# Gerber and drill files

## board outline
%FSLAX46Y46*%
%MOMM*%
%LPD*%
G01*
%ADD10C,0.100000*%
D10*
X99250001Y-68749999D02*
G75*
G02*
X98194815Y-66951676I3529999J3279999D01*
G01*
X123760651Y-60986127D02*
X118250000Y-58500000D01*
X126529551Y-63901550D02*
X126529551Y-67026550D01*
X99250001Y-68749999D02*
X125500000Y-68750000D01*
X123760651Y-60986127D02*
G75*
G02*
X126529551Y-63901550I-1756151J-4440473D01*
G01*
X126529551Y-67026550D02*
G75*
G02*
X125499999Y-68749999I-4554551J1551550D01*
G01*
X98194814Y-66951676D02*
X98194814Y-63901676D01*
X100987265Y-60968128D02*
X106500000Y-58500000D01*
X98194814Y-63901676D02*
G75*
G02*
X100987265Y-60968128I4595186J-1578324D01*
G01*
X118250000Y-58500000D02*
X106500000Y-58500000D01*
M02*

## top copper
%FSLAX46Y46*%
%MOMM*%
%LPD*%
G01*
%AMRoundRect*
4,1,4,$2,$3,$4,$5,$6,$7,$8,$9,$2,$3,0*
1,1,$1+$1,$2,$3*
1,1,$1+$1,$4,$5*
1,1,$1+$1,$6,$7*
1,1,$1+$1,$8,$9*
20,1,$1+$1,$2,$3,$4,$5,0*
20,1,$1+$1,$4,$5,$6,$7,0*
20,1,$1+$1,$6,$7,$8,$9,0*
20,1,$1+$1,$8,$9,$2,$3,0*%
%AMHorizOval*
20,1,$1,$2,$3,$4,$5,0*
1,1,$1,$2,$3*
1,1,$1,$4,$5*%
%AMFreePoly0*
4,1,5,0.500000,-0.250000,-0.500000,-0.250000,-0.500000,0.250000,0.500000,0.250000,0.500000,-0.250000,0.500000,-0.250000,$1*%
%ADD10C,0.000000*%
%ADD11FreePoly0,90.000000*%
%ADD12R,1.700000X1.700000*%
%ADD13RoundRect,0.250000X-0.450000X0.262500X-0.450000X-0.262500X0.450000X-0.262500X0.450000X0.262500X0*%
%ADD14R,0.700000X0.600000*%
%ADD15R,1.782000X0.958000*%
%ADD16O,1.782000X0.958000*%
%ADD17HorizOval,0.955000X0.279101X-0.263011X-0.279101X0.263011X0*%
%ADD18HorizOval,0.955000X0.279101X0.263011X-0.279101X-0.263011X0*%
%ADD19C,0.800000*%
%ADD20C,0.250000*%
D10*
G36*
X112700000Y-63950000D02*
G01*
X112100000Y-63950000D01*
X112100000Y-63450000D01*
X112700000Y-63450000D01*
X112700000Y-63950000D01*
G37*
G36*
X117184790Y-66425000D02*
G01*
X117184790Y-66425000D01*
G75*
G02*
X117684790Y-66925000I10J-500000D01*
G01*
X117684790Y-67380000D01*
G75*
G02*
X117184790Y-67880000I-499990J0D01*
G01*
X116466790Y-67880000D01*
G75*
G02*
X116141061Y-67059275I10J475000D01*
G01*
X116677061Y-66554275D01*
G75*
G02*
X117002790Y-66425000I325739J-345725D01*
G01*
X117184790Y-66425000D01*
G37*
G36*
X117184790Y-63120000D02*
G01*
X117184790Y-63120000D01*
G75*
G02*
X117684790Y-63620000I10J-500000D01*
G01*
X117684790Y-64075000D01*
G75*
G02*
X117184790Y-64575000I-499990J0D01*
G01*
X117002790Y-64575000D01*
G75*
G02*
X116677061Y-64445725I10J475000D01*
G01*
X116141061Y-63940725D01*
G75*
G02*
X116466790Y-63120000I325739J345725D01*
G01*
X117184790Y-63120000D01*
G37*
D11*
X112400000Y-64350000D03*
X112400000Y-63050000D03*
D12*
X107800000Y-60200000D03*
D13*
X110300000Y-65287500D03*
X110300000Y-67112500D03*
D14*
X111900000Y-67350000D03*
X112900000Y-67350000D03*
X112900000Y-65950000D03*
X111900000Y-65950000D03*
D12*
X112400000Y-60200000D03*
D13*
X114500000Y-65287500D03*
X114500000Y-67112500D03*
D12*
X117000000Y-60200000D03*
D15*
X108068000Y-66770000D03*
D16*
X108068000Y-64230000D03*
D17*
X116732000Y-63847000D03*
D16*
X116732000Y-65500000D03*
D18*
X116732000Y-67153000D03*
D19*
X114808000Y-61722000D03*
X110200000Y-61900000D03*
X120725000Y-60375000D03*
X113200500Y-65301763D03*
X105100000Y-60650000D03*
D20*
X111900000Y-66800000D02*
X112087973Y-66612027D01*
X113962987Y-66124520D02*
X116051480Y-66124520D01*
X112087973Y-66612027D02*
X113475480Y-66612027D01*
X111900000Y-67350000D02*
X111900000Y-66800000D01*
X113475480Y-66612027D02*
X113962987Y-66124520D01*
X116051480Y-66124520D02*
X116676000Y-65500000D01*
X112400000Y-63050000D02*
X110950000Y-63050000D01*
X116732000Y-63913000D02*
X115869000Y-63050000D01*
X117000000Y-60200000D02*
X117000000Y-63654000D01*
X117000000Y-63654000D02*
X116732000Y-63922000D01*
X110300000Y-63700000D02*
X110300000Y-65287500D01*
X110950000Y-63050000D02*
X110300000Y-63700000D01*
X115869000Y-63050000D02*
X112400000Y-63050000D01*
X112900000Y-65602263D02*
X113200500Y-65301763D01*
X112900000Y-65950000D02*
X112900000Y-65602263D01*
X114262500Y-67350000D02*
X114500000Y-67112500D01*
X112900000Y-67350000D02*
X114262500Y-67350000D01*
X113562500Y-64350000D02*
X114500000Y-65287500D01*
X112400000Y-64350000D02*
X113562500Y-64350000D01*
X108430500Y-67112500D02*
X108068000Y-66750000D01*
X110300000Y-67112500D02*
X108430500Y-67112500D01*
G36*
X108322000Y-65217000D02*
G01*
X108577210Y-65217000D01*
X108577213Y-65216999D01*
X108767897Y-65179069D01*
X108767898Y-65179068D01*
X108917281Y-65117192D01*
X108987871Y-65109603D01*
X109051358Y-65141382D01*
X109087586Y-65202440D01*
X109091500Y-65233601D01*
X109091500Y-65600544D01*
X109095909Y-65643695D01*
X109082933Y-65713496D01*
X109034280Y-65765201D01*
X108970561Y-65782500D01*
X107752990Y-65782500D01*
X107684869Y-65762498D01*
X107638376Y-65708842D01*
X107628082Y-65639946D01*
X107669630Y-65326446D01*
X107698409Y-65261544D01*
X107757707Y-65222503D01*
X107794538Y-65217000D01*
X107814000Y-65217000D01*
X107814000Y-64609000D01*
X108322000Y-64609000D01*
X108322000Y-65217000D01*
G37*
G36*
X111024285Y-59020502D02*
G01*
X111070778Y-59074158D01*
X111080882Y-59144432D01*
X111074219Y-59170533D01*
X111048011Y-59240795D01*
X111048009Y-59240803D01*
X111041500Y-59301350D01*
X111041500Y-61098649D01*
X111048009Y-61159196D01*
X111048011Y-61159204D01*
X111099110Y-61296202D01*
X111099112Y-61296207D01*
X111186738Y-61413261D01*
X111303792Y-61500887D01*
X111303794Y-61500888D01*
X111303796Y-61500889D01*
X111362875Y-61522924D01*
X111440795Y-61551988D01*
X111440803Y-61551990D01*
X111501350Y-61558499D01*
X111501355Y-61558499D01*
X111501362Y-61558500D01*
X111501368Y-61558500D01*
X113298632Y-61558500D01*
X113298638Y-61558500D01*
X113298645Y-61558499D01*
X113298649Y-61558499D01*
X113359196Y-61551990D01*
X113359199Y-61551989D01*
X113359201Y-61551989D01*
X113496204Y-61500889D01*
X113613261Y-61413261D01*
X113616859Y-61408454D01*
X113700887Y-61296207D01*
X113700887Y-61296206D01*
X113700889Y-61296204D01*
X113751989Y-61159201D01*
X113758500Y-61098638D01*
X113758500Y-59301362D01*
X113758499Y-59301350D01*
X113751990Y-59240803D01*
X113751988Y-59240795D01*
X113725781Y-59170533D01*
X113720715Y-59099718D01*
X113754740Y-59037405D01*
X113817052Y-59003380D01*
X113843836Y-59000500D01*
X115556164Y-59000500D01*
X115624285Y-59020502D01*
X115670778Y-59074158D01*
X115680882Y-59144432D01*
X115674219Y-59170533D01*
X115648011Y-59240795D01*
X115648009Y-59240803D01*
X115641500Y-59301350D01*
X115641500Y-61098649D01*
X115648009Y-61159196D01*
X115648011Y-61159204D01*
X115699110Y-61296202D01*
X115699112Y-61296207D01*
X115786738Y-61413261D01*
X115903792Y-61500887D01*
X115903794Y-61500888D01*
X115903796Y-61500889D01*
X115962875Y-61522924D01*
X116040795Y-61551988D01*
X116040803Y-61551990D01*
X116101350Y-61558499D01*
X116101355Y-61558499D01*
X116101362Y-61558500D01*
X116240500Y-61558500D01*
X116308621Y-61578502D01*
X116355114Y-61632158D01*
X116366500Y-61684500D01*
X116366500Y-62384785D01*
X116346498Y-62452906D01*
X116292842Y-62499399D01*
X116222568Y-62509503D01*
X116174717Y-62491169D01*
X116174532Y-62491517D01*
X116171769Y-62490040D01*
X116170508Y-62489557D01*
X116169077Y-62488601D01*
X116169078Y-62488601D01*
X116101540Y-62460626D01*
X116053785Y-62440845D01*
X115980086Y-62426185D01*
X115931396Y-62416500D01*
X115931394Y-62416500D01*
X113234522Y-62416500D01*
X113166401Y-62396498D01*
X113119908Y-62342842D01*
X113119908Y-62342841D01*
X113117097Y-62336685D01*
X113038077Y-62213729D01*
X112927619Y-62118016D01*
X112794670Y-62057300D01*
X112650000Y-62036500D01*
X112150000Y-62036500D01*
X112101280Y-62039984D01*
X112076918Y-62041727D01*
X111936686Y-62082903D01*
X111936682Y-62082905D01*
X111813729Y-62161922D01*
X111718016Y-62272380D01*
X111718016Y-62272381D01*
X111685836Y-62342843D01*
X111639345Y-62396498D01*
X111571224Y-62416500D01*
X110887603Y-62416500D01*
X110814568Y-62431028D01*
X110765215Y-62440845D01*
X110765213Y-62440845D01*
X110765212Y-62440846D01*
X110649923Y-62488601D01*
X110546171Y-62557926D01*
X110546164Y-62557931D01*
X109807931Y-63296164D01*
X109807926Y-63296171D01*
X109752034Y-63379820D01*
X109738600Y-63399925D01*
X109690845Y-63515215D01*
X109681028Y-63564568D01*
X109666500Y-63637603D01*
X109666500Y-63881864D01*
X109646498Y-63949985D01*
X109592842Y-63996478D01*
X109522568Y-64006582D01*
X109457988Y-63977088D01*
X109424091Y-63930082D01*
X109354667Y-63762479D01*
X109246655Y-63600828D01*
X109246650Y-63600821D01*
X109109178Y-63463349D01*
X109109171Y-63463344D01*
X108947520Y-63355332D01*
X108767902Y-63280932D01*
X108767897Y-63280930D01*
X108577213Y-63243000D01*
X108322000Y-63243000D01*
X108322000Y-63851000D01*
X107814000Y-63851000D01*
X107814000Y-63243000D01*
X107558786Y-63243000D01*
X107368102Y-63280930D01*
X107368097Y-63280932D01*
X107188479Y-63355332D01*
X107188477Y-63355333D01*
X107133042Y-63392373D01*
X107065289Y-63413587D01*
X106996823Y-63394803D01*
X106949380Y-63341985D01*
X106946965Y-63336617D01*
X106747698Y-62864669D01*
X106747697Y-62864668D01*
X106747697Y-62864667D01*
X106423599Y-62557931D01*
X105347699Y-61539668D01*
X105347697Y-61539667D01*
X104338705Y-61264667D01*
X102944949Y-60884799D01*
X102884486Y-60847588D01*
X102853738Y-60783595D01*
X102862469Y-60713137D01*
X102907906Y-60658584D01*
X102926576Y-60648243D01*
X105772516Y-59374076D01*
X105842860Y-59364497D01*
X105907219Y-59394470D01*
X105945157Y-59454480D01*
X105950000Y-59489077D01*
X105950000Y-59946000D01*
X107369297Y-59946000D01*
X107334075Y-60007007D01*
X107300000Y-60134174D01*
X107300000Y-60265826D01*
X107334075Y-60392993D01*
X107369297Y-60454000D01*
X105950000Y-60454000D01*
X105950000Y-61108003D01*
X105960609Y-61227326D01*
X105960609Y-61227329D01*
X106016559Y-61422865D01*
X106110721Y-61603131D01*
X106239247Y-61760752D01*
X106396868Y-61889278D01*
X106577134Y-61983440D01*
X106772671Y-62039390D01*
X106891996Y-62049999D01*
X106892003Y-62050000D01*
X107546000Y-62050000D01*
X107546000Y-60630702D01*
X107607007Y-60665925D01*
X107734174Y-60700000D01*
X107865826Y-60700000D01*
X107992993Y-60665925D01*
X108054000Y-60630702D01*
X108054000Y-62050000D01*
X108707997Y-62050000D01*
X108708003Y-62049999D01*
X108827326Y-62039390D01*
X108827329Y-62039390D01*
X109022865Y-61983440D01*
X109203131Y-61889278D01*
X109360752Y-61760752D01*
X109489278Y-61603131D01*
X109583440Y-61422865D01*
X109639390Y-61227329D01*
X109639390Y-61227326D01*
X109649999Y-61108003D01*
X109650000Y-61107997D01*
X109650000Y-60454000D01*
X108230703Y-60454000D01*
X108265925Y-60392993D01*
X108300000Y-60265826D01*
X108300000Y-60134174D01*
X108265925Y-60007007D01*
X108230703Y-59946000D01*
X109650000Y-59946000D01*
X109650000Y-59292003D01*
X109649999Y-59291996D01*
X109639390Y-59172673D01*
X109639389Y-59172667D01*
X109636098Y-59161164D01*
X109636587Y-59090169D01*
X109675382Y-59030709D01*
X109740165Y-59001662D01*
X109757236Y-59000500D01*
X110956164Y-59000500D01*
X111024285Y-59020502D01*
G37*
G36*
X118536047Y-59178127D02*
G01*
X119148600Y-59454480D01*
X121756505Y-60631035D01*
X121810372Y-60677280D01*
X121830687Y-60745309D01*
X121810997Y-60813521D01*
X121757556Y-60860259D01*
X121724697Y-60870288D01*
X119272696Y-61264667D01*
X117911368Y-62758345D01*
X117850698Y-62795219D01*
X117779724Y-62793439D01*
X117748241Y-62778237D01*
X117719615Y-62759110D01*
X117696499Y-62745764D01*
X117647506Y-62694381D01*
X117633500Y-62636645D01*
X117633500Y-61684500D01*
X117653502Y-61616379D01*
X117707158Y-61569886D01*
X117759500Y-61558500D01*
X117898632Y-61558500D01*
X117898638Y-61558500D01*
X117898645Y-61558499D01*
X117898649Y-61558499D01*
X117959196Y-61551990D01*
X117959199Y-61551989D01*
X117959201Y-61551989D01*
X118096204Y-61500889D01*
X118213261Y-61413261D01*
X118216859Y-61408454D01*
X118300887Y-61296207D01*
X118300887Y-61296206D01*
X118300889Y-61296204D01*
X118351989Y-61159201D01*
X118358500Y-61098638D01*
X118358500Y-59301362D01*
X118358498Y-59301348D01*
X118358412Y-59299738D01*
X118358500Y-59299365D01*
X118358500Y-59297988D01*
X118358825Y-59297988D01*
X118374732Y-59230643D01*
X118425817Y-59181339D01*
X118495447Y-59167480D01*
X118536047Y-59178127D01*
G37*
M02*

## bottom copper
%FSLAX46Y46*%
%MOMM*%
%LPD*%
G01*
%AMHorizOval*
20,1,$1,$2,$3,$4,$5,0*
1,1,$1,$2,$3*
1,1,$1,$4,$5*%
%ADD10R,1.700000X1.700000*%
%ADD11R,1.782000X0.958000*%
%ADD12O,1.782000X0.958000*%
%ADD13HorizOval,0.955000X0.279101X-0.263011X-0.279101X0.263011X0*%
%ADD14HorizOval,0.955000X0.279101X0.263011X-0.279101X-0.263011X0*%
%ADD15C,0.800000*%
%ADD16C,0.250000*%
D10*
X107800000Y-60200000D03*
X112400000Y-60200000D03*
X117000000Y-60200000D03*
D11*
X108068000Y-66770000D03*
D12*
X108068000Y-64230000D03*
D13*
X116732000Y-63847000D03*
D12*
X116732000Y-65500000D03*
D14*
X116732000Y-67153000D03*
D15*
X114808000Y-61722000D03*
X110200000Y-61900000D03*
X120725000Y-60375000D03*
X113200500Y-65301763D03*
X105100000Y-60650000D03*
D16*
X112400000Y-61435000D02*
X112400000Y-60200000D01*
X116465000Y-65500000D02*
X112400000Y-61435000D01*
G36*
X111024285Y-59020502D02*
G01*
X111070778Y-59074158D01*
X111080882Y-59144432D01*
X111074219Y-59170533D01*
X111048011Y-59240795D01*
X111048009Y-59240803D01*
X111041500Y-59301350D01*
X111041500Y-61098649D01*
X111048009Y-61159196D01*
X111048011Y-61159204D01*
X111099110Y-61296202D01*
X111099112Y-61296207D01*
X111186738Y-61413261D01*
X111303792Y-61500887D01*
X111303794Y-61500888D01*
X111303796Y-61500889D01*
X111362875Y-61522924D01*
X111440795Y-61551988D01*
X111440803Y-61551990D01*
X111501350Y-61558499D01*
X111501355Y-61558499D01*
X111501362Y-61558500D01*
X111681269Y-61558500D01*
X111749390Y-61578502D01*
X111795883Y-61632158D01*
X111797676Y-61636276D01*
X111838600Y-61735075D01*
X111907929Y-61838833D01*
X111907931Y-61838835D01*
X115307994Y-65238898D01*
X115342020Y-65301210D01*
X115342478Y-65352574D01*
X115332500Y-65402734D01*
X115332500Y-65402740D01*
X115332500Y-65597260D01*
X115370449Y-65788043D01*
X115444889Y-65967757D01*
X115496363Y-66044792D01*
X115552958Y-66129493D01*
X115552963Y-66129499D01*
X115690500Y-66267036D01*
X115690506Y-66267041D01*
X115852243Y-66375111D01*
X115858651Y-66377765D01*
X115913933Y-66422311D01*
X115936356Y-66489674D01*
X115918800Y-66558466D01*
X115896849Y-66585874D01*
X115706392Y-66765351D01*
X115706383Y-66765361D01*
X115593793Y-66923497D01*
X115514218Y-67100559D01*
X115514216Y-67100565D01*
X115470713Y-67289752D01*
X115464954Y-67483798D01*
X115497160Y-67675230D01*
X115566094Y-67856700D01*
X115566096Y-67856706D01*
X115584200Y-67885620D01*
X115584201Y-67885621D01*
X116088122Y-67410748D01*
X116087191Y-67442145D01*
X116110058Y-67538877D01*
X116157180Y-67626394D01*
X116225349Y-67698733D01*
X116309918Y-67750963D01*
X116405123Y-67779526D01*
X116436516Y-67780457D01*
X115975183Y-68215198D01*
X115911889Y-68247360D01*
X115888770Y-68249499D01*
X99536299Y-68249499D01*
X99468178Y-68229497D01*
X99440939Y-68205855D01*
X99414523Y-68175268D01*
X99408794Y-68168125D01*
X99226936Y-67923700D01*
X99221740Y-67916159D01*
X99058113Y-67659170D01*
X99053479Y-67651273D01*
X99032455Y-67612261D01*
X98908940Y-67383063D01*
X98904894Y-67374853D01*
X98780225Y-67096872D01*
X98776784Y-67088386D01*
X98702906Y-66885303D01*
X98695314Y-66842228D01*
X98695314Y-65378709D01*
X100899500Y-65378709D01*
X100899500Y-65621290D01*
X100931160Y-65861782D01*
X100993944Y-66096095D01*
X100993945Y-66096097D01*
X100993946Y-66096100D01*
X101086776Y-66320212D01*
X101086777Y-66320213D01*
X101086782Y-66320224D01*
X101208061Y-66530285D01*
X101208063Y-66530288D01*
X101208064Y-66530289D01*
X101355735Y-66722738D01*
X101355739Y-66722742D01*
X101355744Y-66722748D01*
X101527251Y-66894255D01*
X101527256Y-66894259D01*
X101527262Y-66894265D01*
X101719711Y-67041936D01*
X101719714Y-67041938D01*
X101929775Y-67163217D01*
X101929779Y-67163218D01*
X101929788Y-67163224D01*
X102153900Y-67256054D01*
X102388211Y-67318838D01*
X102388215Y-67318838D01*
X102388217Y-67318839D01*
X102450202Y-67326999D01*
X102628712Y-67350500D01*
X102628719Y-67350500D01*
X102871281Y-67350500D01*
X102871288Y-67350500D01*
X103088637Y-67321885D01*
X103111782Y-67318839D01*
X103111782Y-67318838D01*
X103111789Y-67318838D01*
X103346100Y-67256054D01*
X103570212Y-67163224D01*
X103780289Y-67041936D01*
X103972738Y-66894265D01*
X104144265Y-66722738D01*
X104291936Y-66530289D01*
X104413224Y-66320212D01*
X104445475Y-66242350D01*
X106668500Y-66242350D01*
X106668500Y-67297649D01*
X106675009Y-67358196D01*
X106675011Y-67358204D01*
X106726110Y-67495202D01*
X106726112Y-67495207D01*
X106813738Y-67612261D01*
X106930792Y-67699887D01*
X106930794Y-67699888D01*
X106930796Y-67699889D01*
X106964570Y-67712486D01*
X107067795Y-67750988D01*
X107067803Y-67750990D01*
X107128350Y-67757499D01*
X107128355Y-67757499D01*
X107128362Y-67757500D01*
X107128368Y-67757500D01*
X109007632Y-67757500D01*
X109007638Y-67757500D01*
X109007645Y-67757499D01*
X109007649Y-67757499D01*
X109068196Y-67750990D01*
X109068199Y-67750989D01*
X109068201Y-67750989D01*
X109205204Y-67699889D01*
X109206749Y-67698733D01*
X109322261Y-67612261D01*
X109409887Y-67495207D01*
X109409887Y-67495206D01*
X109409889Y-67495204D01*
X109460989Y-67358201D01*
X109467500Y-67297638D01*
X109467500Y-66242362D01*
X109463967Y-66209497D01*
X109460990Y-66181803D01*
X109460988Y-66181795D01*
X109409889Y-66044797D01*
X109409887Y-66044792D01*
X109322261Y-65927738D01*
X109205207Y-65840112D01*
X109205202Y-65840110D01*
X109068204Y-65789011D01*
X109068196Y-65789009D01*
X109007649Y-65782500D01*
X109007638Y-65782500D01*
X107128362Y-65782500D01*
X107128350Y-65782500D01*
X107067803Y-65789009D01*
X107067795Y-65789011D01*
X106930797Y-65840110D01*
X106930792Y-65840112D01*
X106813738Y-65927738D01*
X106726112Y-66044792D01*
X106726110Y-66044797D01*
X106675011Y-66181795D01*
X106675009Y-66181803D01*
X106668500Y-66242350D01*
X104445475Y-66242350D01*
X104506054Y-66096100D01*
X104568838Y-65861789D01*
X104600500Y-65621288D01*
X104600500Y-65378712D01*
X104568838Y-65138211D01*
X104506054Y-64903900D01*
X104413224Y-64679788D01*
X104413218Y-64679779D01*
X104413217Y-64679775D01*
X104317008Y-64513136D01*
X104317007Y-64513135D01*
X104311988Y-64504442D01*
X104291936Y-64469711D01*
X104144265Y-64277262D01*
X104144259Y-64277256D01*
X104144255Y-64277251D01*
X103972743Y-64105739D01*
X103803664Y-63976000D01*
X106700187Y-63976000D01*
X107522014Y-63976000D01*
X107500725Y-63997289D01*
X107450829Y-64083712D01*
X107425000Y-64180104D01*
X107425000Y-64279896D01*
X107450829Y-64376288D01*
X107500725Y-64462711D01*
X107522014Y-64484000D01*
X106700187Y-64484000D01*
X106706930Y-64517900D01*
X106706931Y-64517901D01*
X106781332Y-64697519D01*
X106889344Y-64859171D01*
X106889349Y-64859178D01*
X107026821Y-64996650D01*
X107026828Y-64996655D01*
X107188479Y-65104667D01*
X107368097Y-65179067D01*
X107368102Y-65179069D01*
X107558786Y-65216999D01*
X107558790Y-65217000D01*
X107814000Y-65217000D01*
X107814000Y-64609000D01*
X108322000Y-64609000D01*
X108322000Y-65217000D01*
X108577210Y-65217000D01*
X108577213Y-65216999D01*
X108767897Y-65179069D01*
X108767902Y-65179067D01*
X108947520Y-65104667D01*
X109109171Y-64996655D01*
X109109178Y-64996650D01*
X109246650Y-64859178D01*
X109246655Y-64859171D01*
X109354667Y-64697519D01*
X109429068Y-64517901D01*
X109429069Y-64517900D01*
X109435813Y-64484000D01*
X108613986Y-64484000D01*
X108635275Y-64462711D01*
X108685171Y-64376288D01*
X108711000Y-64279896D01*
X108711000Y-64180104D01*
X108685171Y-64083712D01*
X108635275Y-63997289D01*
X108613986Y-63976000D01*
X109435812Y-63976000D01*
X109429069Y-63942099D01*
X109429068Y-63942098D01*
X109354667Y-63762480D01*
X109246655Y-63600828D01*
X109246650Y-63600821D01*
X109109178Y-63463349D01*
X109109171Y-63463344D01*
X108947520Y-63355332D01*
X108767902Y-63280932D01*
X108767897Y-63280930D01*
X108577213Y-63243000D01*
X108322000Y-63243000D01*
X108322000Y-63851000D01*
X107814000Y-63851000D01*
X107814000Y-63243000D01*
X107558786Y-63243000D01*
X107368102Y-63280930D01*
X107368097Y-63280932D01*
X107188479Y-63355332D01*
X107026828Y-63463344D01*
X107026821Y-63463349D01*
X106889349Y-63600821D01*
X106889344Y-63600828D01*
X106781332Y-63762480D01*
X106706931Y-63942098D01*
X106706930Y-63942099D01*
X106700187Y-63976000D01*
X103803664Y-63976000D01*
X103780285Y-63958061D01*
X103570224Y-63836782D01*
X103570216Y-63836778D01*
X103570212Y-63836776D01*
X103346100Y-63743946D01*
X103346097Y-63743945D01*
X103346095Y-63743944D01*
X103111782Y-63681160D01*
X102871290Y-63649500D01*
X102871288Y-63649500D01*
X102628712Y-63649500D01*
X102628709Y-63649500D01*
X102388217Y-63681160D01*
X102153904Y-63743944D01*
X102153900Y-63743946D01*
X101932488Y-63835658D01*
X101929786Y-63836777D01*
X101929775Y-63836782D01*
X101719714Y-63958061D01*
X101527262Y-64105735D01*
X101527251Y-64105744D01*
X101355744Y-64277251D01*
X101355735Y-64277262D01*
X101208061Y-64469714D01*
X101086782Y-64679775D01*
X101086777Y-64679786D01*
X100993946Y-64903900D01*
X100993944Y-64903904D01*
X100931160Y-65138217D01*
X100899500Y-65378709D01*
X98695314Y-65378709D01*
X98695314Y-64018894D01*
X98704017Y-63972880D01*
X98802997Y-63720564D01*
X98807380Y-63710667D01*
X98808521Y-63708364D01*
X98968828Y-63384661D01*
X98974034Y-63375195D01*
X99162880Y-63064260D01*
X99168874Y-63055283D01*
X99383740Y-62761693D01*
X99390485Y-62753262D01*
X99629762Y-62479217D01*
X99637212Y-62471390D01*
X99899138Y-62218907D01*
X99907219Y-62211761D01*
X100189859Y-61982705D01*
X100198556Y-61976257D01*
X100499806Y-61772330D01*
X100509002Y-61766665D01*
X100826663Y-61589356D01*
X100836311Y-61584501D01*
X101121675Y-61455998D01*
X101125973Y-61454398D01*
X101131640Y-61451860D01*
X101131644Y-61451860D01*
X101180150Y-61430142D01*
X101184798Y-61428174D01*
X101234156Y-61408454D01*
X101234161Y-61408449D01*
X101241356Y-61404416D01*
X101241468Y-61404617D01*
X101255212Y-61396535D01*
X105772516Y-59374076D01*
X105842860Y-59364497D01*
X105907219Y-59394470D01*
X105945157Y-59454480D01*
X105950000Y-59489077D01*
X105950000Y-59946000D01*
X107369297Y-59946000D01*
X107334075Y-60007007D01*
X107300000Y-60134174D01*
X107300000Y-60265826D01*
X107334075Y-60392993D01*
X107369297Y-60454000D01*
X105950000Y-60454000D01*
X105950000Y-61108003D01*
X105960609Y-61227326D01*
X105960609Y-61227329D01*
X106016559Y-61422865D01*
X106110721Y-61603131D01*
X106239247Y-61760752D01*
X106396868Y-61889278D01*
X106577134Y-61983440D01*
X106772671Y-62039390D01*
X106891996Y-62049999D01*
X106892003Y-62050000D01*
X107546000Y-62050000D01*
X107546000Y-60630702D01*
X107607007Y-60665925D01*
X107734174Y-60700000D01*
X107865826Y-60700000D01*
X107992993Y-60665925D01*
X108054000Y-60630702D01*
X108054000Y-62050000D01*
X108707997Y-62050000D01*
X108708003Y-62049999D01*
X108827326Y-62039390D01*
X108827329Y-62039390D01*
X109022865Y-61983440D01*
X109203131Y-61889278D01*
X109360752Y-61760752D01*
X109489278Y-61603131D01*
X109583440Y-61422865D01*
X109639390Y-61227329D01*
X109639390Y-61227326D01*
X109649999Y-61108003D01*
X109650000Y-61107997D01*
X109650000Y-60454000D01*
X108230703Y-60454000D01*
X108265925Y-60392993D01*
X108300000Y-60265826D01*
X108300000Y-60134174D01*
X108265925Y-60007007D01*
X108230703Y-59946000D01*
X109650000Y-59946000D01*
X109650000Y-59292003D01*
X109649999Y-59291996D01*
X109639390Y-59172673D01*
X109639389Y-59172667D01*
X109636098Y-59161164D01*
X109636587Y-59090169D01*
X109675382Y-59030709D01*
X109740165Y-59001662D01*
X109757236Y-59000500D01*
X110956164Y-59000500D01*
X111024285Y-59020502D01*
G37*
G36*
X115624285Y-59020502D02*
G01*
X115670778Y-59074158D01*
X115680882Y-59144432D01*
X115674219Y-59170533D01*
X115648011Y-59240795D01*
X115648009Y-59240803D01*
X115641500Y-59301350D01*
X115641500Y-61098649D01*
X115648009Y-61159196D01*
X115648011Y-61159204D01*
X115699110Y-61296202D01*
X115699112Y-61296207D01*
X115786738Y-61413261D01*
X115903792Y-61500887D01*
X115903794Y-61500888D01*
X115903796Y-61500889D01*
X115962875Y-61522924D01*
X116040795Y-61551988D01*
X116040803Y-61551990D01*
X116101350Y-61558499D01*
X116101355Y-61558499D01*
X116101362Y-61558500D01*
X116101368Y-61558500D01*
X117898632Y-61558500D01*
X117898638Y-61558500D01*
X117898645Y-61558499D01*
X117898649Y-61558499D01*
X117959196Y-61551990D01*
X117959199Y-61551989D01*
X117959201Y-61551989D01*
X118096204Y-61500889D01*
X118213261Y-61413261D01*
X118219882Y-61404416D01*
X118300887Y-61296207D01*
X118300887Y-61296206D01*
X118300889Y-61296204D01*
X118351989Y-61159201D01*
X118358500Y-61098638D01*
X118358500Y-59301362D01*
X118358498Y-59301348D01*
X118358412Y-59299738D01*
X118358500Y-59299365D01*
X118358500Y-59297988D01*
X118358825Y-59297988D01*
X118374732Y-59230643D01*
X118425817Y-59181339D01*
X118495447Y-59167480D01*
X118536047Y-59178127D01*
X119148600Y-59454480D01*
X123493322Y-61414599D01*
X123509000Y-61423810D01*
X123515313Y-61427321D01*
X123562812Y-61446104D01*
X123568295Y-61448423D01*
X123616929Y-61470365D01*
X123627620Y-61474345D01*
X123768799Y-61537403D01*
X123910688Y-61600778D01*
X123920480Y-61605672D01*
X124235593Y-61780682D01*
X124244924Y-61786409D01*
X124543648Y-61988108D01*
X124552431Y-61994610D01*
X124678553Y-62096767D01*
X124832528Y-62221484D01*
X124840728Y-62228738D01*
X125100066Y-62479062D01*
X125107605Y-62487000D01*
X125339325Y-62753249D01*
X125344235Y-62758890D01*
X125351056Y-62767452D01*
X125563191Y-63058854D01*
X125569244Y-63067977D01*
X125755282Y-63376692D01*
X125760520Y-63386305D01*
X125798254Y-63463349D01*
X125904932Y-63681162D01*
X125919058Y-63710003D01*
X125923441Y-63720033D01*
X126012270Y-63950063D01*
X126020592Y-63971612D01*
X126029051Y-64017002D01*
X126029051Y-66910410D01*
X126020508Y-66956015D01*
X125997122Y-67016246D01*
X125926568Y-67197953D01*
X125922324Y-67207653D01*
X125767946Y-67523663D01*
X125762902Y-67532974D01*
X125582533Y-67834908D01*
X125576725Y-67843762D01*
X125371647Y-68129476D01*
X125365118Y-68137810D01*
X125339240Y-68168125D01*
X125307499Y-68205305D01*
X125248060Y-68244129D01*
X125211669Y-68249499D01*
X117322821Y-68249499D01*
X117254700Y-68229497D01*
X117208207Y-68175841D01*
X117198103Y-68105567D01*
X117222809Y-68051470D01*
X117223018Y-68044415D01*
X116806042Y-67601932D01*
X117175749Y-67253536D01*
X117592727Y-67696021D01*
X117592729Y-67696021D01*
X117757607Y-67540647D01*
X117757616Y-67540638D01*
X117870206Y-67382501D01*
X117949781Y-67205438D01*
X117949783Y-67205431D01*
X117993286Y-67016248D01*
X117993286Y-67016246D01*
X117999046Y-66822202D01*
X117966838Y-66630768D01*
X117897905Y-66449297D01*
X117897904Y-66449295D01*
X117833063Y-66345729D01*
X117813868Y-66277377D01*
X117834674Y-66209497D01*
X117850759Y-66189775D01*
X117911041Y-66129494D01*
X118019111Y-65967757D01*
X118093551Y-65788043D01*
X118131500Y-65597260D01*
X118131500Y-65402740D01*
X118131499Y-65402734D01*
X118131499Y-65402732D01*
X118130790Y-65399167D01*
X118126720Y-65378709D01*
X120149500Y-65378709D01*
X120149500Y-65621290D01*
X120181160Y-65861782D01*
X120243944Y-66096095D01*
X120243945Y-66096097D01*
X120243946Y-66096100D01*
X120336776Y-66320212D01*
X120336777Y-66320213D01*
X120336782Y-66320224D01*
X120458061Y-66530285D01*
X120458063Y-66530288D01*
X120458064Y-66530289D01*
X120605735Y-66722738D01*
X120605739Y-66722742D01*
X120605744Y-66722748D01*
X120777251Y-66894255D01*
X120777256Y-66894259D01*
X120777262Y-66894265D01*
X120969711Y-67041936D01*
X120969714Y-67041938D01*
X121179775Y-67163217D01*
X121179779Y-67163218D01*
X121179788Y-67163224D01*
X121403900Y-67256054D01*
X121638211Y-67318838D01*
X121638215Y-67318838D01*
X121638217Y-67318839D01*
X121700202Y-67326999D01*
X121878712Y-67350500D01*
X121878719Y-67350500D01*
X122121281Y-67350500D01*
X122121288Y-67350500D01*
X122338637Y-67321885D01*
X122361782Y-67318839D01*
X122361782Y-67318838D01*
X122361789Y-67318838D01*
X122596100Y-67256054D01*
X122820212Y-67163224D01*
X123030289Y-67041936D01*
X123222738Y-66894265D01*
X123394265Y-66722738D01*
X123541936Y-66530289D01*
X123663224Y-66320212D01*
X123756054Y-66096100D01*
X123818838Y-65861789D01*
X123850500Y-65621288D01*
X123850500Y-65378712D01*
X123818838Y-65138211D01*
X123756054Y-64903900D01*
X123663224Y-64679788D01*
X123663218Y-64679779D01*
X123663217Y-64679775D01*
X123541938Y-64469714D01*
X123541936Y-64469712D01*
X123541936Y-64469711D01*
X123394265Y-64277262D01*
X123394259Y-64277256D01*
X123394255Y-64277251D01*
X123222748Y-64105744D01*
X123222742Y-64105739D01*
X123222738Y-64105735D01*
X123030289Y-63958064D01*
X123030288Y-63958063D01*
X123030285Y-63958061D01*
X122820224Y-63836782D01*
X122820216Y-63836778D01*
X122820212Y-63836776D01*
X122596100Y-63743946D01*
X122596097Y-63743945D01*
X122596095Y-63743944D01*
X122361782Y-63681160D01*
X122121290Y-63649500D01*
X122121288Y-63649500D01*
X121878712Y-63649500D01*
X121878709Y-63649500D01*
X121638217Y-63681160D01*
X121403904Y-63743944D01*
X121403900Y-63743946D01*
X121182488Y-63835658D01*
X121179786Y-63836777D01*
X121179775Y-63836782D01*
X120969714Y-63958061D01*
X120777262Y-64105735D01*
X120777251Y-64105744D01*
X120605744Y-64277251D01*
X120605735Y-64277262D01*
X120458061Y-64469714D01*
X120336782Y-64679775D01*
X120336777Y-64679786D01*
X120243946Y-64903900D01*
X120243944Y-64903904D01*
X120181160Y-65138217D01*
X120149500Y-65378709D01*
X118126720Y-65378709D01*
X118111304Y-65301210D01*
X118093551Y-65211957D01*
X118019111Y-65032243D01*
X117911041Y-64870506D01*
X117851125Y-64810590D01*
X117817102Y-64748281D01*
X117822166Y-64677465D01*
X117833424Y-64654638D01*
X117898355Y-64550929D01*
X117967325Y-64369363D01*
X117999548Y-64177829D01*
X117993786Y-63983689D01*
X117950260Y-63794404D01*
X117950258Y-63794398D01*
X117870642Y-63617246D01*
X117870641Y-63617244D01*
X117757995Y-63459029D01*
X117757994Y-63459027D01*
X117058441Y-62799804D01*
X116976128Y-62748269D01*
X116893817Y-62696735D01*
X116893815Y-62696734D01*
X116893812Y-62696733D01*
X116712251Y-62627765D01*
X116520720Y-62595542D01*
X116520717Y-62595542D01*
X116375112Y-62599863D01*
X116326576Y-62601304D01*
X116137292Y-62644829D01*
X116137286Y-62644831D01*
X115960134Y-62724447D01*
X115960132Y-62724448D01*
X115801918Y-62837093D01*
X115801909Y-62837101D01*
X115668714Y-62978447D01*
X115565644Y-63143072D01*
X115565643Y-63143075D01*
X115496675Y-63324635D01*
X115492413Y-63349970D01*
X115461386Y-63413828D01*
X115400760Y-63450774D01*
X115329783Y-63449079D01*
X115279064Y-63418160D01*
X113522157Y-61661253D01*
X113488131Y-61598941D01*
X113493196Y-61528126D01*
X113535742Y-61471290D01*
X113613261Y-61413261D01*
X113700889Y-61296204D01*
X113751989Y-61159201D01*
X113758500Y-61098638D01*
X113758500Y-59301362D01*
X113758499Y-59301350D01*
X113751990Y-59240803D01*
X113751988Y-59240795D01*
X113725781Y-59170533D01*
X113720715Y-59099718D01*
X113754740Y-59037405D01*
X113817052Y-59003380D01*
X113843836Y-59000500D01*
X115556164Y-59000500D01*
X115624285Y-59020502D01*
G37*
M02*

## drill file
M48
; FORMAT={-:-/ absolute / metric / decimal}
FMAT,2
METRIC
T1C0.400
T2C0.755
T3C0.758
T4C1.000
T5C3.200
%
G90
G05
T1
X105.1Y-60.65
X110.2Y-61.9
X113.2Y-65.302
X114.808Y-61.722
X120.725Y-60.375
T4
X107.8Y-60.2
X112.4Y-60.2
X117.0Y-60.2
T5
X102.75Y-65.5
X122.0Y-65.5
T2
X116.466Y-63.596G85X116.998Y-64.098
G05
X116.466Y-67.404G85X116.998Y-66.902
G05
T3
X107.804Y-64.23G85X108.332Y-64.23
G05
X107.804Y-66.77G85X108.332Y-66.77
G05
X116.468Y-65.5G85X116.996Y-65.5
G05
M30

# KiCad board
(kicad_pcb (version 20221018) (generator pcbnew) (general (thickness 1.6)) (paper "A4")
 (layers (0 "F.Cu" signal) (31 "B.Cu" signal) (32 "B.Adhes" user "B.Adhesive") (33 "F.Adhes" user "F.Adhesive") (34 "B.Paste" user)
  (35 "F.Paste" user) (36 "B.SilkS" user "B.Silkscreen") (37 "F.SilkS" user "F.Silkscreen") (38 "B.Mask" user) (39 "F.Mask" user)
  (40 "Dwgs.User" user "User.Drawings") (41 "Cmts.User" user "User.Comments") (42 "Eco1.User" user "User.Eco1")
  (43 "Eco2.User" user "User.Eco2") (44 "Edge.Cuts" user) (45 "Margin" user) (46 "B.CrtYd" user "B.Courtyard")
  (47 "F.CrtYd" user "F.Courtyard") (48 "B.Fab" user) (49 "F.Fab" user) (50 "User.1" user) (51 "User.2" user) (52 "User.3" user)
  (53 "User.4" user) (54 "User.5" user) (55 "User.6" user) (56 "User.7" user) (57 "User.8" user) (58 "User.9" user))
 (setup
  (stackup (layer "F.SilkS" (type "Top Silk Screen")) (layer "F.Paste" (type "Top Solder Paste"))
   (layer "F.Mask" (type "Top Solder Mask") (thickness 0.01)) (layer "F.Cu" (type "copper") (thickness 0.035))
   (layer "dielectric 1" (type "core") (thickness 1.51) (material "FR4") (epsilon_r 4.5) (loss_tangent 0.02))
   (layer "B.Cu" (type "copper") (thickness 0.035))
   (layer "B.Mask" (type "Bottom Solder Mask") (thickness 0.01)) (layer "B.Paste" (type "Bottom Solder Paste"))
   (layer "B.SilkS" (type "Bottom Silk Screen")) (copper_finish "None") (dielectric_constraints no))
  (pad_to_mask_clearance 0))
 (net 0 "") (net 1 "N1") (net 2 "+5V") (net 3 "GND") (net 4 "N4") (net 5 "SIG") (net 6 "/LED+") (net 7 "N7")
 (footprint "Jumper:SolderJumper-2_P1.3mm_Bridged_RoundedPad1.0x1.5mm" (layer "F.Cu") (at 112.4 63.7 90) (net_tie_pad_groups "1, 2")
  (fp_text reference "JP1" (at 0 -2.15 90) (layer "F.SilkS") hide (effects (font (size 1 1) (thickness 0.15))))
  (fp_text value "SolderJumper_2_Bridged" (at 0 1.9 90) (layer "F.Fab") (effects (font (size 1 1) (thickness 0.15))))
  (fp_poly (pts (xy 0.25 -0.3) (xy -0.25 -0.3) (xy -0.25 0.3) (xy 0.25 0.3)) (stroke (width 0) (type solid)) (fill solid) (layer "F.Cu"))
  (pad "1" smd custom (at -0.65 0 90) (size 1 0.5) (layers "F.Cu" "F.Mask") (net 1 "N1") (zone_connect 2) (thermal_bridge_angle 45)
   (options (clearance outline) (anchor rect)) (primitives))
  (pad "2" smd custom (at 0.65 0 90) (size 1 0.5) (layers "F.Cu" "F.Mask") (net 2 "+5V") (zone_connect 2) (thermal_bridge_angle 45)
   (options (clearance outline) (anchor rect)) (primitives)))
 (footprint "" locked (layer "F.Cu") (at 122 65.5)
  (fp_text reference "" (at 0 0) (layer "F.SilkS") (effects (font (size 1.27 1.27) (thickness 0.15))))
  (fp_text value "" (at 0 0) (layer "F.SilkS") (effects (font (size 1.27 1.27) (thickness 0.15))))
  (pad "" np_thru_hole circle locked (at 0 0) (size 3.2 3.2) (drill 3.2) (layers "*.Cu" "*.Mask")))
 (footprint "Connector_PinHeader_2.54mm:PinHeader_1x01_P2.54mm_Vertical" (layer "F.Cu") (at 107.8 60.2)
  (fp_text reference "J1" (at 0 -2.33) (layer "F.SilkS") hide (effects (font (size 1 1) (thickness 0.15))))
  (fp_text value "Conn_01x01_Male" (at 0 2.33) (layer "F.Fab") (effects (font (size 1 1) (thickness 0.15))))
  (pad "1" thru_hole rect (at 0 0) (size 1.7 1.7) (drill 1) (layers "*.Cu" "*.Mask") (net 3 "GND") (thermal_gap 1)))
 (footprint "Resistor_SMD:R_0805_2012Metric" (layer "F.Cu") (at 110.3 66.2 -90)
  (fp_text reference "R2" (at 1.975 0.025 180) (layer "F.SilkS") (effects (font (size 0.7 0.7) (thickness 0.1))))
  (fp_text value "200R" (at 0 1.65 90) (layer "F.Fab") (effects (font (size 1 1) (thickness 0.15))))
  (pad "1" smd roundrect (at -0.9125 0 270) (size 1.025 1.4) (layers "F.Cu" "F.Paste" "F.Mask") (roundrect_rratio 0.243902439) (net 2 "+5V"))
  (pad "2" smd roundrect (at 0.9125 0 270) (size 1.025 1.4) (layers "F.Cu" "F.Paste" "F.Mask") (roundrect_rratio 0.243902439) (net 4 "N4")))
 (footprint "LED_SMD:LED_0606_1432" (layer "F.Cu") (at 112.4 66.65 90)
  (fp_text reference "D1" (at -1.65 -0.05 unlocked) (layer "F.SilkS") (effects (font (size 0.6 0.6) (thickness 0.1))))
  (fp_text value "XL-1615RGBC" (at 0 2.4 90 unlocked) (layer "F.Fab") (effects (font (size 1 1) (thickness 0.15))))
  (pad "1" smd rect (at -0.7 -0.5 90) (size 0.6 0.7) (layers "F.Cu" "F.Paste" "F.Mask") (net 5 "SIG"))
  (pad "2" smd rect (at -0.7 0.5 90) (size 0.6 0.7) (layers "F.Cu" "F.Paste" "F.Mask") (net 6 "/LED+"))
  (pad "3" smd rect (at 0.7 0.5 90) (size 0.6 0.7) (layers "F.Cu" "F.Paste" "F.Mask") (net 3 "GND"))
  (pad "4" smd rect (at 0.7 -0.5 90) (size 0.6 0.7) (layers "F.Cu" "F.Paste" "F.Mask") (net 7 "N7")))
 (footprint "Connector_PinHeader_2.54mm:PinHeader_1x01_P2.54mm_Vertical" (layer "F.Cu") (at 112.4 60.2)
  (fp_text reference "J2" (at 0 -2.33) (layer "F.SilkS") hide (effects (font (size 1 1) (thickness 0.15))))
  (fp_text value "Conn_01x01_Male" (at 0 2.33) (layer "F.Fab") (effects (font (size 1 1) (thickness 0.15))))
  (pad "1" thru_hole rect (at 0 0) (size 1.7 1.7) (drill 1) (layers "*.Cu" "*.Mask") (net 5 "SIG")))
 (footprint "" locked (layer "F.Cu") (at 102.75 65.5)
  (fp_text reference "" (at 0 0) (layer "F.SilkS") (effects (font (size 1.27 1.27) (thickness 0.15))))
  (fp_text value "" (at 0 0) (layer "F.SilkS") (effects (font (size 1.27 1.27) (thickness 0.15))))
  (pad "" np_thru_hole circle locked (at 0 0) (size 3.2 3.2) (drill 3.2) (layers "*.Cu" "*.Mask")))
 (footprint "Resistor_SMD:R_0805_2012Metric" (layer "F.Cu") (at 114.5 66.2 -90)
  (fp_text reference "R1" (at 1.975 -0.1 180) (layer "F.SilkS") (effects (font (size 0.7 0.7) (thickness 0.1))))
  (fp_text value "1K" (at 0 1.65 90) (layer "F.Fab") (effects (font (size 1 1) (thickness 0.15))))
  (pad "1" smd roundrect (at -0.9125 0 270) (size 1.025 1.4) (layers "F.Cu" "F.Paste" "F.Mask") (roundrect_rratio 0.243902439) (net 1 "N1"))
  (pad "2" smd roundrect (at 0.9125 0 270) (size 1.025 1.4) (layers "F.Cu" "F.Paste" "F.Mask") (roundrect_rratio 0.243902439)
   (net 6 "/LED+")))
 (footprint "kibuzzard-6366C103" (layer "F.Cu") (at 122.35 62.1 -25)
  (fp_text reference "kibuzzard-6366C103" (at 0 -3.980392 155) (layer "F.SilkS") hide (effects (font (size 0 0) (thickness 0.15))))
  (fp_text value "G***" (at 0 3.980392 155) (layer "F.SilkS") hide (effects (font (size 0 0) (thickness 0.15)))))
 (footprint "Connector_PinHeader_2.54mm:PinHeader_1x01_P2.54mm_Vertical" (layer "F.Cu") (at 117 60.2)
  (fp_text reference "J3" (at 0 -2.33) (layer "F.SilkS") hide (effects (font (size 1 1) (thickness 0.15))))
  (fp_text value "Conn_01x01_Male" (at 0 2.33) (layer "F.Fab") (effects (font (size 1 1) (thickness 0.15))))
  (pad "1" thru_hole rect (at 0 0) (size 1.7 1.7) (drill 1) (layers "*.Cu" "*.Mask") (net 2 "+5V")))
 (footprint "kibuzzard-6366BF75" (layer "B.Cu") (at 122.302977 62.093652 155)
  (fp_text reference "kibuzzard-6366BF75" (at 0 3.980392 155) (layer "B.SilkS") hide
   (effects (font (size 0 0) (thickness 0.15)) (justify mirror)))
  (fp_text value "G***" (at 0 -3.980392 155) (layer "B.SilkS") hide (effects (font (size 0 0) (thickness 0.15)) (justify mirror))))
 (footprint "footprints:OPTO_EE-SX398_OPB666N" (layer "B.Cu") (at 112.4 65.5 180)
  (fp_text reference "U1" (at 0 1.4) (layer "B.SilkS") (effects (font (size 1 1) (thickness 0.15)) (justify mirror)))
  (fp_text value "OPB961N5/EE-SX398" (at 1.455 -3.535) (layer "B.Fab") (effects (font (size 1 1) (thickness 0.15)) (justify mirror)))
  (fp_poly
   (pts
    (arc (start -4.06679 -2.38) (mid -3.62529 -2.080222) (end -3.741061 -1.559275))
    (arc (start -4.277061 -1.054275) (mid -4.427568 -0.9585) (end -4.60279 -0.925))
    (arc (start -4.78479 -0.925) (mid -5.138343 -1.071447) (end -5.28479 -1.425))
    (arc (start -5.28479 -1.88) (mid -5.138343 -2.233553) (end -4.78479 -2.38)))
   (stroke (width 0) (type solid)) (fill solid) (layer "F.Cu"))
  (fp_poly
   (pts
    (arc (start -3.741061 1.559275) (mid -3.62529 2.080222) (end -4.06679 2.38))
    (arc (start -4.78479 2.38) (mid -5.138343 2.233553) (end -5.28479 1.88))
    (arc (start -5.28479 1.425) (mid -5.138343 1.071447) (end -4.78479 0.925))
    (arc (start -4.60279 0.925) (mid -4.427568 0.9585) (end -4.277061 1.054275)))
   (stroke (width 0) (type solid)) (fill solid) (layer "F.Cu"))
  (pad "1" thru_hole rect (at 4.332 -1.27) (size 1.782 0.958) (drill oval 1.286 0.758) (layers "*.Cu" "*.Mask") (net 4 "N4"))
  (pad "2" thru_hole oval (at 4.332 1.27) (size 1.782 0.958) (drill oval 1.286 0.758) (layers "*.Cu" "*.Mask") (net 3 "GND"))
  (pad "3" thru_hole oval (at -4.332 1.653 316.7) (size 1.722 0.955) (drill oval 1.486 0.755) (layers "*.Cu" "*.Mask") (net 2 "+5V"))
  (pad "4" thru_hole oval (at -4.332 0) (size 1.782 0.958) (drill oval 1.286 0.758) (layers "*.Cu" "*.Mask") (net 5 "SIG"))
  (pad "5" thru_hole oval (at -4.332 -1.653 43.3) (size 1.722 0.955) (drill oval 1.486 0.755) (layers "*.Cu" "*.Mask") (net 3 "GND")))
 (gr_arc (start 99.250001 68.749999) (mid 98.623975 67.908594) (end 98.194814 66.951676) (stroke (width 0.1) (type default))
  (layer "Edge.Cuts"))
 (gr_line (start 123.760651 60.986127) (end 118.25 58.5) (stroke (width 0.1) (type solid)) (layer "Edge.Cuts"))
 (gr_line (start 126.529551 63.90155) (end 126.529551 67.02655) (stroke (width 0.1) (type default)) (layer "Edge.Cuts"))
 (gr_line (start 99.250001 68.749999) (end 125.5 68.75) (stroke (width 0.1) (type solid)) (layer "Edge.Cuts"))
 (gr_arc (start 123.760651 60.986127) (mid 125.466917 62.138197) (end 126.529551 63.90155) (stroke (width 0.1) (type solid))
  (layer "Edge.Cuts"))
 (gr_arc (start 126.529551 67.02655) (mid 126.10566 67.942567) (end 125.5 68.75) (stroke (width 0.1) (type solid)) (layer "Edge.Cuts"))
 (gr_line (start 98.194814 66.951676) (end 98.194814 63.901676) (stroke (width 0.1) (type default)) (layer "Edge.Cuts"))
 (gr_line (start 100.987265 60.968128) (end 106.5 58.5) (stroke (width 0.1) (type solid)) (layer "Edge.Cuts"))
 (gr_arc (start 98.194814 63.901676) (mid 99.270799 62.130065) (end 100.987265 60.968128) (stroke (width 0.1) (type default))
  (layer "Edge.Cuts"))
 (gr_line (start 118.25 58.5) (end 106.5 58.5) (stroke (width 0.1) (type solid)) (layer "Edge.Cuts"))
 (segment (start 111.9 66.8) (end 112.087973 66.612027) (width 0.25) (layer "F.Cu") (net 5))
 (segment (start 113.962987 66.12452) (end 116.05148 66.12452) (width 0.25) (layer "F.Cu") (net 5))
 (segment (start 112.087973 66.612027) (end 113.47548 66.612027) (width 0.25) (layer "F.Cu") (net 5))
 (segment (start 111.9 67.35) (end 111.9 66.8) (width 0.25) (layer "F.Cu") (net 5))
 (segment (start 113.47548 66.612027) (end 113.962987 66.12452) (width 0.25) (layer "F.Cu") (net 5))
 (segment (start 116.05148 66.12452) (end 116.676 65.5) (width 0.25) (layer "F.Cu") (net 5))
 (segment (start 112.4 61.435) (end 112.4 60.2) (width 0.25) (layer "B.Cu") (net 5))
 (segment (start 116.465 65.5) (end 112.4 61.435) (width 0.25) (layer "B.Cu") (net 5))
 (segment (start 112.4 63.05) (end 110.95 63.05) (width 0.25) (layer "F.Cu") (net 2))
 (segment (start 116.732 63.913) (end 115.869 63.05) (width 0.25) (layer "F.Cu") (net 2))
 (segment (start 117 60.2) (end 117 63.654) (width 0.25) (layer "F.Cu") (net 2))
 (segment (start 117 63.654) (end 116.732 63.922) (width 0.25) (layer "F.Cu") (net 2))
 (segment (start 110.3 63.7) (end 110.3 65.2875) (width 0.25) (layer "F.Cu") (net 2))
 (segment (start 110.95 63.05) (end 110.3 63.7) (width 0.25) (layer "F.Cu") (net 2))
 (segment (start 115.869 63.05) (end 112.4 63.05) (width 0.25) (layer "F.Cu") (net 2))
 (segment (start 112.9 65.602263) (end 113.2005 65.301763) (width 0.25) (layer "F.Cu") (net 3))
 (segment (start 112.9 65.95) (end 112.9 65.602263) (width 0.25) (layer "F.Cu") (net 3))
 (via (at 114.808 61.722) (size 0.8) (drill 0.4) (layers "F.Cu" "B.Cu") (free) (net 3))
 (via (at 110.2 61.9) (size 0.8) (drill 0.4) (layers "F.Cu" "B.Cu") (free) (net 3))
 (via (at 120.725 60.375) (size 0.8) (drill 0.4) (layers "F.Cu" "B.Cu") (free) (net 3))
 (via (at 113.2005 65.301763) (size 0.8) (drill 0.4) (layers "F.Cu" "B.Cu") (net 3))
 (via (at 105.1 60.65) (size 0.8) (drill 0.4) (layers "F.Cu" "B.Cu") (free) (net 3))
 (segment (start 114.2625 67.35) (end 114.5 67.1125) (width 0.25) (layer "F.Cu") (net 6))
 (segment (start 112.9 67.35) (end 114.2625 67.35) (width 0.25) (layer "F.Cu") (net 6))
 (segment (start 113.5625 64.35) (end 114.5 65.2875) (width 0.25) (layer "F.Cu") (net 1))
 (segment (start 112.4 64.35) (end 113.5625 64.35) (width 0.25) (layer "F.Cu") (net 1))
 (segment (start 108.4305 67.1125) (end 108.068 66.75) (width 0.25) (layer "F.Cu") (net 4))
 (segment (start 110.3 67.1125) (end 108.4305 67.1125) (width 0.25) (layer "F.Cu") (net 4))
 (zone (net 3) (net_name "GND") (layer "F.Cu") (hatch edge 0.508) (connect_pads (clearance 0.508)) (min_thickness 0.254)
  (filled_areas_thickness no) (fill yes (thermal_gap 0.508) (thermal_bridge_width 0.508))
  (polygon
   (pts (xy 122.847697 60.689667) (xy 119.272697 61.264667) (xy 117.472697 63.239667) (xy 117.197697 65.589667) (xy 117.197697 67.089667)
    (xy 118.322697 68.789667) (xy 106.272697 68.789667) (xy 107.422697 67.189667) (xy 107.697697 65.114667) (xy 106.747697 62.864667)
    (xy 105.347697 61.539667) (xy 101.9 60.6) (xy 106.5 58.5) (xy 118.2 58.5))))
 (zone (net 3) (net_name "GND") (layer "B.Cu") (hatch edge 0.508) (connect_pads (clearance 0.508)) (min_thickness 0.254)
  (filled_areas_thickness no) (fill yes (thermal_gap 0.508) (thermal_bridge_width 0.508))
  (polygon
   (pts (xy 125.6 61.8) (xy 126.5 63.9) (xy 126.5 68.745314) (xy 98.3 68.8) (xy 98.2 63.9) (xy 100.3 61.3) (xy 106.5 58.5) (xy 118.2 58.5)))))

